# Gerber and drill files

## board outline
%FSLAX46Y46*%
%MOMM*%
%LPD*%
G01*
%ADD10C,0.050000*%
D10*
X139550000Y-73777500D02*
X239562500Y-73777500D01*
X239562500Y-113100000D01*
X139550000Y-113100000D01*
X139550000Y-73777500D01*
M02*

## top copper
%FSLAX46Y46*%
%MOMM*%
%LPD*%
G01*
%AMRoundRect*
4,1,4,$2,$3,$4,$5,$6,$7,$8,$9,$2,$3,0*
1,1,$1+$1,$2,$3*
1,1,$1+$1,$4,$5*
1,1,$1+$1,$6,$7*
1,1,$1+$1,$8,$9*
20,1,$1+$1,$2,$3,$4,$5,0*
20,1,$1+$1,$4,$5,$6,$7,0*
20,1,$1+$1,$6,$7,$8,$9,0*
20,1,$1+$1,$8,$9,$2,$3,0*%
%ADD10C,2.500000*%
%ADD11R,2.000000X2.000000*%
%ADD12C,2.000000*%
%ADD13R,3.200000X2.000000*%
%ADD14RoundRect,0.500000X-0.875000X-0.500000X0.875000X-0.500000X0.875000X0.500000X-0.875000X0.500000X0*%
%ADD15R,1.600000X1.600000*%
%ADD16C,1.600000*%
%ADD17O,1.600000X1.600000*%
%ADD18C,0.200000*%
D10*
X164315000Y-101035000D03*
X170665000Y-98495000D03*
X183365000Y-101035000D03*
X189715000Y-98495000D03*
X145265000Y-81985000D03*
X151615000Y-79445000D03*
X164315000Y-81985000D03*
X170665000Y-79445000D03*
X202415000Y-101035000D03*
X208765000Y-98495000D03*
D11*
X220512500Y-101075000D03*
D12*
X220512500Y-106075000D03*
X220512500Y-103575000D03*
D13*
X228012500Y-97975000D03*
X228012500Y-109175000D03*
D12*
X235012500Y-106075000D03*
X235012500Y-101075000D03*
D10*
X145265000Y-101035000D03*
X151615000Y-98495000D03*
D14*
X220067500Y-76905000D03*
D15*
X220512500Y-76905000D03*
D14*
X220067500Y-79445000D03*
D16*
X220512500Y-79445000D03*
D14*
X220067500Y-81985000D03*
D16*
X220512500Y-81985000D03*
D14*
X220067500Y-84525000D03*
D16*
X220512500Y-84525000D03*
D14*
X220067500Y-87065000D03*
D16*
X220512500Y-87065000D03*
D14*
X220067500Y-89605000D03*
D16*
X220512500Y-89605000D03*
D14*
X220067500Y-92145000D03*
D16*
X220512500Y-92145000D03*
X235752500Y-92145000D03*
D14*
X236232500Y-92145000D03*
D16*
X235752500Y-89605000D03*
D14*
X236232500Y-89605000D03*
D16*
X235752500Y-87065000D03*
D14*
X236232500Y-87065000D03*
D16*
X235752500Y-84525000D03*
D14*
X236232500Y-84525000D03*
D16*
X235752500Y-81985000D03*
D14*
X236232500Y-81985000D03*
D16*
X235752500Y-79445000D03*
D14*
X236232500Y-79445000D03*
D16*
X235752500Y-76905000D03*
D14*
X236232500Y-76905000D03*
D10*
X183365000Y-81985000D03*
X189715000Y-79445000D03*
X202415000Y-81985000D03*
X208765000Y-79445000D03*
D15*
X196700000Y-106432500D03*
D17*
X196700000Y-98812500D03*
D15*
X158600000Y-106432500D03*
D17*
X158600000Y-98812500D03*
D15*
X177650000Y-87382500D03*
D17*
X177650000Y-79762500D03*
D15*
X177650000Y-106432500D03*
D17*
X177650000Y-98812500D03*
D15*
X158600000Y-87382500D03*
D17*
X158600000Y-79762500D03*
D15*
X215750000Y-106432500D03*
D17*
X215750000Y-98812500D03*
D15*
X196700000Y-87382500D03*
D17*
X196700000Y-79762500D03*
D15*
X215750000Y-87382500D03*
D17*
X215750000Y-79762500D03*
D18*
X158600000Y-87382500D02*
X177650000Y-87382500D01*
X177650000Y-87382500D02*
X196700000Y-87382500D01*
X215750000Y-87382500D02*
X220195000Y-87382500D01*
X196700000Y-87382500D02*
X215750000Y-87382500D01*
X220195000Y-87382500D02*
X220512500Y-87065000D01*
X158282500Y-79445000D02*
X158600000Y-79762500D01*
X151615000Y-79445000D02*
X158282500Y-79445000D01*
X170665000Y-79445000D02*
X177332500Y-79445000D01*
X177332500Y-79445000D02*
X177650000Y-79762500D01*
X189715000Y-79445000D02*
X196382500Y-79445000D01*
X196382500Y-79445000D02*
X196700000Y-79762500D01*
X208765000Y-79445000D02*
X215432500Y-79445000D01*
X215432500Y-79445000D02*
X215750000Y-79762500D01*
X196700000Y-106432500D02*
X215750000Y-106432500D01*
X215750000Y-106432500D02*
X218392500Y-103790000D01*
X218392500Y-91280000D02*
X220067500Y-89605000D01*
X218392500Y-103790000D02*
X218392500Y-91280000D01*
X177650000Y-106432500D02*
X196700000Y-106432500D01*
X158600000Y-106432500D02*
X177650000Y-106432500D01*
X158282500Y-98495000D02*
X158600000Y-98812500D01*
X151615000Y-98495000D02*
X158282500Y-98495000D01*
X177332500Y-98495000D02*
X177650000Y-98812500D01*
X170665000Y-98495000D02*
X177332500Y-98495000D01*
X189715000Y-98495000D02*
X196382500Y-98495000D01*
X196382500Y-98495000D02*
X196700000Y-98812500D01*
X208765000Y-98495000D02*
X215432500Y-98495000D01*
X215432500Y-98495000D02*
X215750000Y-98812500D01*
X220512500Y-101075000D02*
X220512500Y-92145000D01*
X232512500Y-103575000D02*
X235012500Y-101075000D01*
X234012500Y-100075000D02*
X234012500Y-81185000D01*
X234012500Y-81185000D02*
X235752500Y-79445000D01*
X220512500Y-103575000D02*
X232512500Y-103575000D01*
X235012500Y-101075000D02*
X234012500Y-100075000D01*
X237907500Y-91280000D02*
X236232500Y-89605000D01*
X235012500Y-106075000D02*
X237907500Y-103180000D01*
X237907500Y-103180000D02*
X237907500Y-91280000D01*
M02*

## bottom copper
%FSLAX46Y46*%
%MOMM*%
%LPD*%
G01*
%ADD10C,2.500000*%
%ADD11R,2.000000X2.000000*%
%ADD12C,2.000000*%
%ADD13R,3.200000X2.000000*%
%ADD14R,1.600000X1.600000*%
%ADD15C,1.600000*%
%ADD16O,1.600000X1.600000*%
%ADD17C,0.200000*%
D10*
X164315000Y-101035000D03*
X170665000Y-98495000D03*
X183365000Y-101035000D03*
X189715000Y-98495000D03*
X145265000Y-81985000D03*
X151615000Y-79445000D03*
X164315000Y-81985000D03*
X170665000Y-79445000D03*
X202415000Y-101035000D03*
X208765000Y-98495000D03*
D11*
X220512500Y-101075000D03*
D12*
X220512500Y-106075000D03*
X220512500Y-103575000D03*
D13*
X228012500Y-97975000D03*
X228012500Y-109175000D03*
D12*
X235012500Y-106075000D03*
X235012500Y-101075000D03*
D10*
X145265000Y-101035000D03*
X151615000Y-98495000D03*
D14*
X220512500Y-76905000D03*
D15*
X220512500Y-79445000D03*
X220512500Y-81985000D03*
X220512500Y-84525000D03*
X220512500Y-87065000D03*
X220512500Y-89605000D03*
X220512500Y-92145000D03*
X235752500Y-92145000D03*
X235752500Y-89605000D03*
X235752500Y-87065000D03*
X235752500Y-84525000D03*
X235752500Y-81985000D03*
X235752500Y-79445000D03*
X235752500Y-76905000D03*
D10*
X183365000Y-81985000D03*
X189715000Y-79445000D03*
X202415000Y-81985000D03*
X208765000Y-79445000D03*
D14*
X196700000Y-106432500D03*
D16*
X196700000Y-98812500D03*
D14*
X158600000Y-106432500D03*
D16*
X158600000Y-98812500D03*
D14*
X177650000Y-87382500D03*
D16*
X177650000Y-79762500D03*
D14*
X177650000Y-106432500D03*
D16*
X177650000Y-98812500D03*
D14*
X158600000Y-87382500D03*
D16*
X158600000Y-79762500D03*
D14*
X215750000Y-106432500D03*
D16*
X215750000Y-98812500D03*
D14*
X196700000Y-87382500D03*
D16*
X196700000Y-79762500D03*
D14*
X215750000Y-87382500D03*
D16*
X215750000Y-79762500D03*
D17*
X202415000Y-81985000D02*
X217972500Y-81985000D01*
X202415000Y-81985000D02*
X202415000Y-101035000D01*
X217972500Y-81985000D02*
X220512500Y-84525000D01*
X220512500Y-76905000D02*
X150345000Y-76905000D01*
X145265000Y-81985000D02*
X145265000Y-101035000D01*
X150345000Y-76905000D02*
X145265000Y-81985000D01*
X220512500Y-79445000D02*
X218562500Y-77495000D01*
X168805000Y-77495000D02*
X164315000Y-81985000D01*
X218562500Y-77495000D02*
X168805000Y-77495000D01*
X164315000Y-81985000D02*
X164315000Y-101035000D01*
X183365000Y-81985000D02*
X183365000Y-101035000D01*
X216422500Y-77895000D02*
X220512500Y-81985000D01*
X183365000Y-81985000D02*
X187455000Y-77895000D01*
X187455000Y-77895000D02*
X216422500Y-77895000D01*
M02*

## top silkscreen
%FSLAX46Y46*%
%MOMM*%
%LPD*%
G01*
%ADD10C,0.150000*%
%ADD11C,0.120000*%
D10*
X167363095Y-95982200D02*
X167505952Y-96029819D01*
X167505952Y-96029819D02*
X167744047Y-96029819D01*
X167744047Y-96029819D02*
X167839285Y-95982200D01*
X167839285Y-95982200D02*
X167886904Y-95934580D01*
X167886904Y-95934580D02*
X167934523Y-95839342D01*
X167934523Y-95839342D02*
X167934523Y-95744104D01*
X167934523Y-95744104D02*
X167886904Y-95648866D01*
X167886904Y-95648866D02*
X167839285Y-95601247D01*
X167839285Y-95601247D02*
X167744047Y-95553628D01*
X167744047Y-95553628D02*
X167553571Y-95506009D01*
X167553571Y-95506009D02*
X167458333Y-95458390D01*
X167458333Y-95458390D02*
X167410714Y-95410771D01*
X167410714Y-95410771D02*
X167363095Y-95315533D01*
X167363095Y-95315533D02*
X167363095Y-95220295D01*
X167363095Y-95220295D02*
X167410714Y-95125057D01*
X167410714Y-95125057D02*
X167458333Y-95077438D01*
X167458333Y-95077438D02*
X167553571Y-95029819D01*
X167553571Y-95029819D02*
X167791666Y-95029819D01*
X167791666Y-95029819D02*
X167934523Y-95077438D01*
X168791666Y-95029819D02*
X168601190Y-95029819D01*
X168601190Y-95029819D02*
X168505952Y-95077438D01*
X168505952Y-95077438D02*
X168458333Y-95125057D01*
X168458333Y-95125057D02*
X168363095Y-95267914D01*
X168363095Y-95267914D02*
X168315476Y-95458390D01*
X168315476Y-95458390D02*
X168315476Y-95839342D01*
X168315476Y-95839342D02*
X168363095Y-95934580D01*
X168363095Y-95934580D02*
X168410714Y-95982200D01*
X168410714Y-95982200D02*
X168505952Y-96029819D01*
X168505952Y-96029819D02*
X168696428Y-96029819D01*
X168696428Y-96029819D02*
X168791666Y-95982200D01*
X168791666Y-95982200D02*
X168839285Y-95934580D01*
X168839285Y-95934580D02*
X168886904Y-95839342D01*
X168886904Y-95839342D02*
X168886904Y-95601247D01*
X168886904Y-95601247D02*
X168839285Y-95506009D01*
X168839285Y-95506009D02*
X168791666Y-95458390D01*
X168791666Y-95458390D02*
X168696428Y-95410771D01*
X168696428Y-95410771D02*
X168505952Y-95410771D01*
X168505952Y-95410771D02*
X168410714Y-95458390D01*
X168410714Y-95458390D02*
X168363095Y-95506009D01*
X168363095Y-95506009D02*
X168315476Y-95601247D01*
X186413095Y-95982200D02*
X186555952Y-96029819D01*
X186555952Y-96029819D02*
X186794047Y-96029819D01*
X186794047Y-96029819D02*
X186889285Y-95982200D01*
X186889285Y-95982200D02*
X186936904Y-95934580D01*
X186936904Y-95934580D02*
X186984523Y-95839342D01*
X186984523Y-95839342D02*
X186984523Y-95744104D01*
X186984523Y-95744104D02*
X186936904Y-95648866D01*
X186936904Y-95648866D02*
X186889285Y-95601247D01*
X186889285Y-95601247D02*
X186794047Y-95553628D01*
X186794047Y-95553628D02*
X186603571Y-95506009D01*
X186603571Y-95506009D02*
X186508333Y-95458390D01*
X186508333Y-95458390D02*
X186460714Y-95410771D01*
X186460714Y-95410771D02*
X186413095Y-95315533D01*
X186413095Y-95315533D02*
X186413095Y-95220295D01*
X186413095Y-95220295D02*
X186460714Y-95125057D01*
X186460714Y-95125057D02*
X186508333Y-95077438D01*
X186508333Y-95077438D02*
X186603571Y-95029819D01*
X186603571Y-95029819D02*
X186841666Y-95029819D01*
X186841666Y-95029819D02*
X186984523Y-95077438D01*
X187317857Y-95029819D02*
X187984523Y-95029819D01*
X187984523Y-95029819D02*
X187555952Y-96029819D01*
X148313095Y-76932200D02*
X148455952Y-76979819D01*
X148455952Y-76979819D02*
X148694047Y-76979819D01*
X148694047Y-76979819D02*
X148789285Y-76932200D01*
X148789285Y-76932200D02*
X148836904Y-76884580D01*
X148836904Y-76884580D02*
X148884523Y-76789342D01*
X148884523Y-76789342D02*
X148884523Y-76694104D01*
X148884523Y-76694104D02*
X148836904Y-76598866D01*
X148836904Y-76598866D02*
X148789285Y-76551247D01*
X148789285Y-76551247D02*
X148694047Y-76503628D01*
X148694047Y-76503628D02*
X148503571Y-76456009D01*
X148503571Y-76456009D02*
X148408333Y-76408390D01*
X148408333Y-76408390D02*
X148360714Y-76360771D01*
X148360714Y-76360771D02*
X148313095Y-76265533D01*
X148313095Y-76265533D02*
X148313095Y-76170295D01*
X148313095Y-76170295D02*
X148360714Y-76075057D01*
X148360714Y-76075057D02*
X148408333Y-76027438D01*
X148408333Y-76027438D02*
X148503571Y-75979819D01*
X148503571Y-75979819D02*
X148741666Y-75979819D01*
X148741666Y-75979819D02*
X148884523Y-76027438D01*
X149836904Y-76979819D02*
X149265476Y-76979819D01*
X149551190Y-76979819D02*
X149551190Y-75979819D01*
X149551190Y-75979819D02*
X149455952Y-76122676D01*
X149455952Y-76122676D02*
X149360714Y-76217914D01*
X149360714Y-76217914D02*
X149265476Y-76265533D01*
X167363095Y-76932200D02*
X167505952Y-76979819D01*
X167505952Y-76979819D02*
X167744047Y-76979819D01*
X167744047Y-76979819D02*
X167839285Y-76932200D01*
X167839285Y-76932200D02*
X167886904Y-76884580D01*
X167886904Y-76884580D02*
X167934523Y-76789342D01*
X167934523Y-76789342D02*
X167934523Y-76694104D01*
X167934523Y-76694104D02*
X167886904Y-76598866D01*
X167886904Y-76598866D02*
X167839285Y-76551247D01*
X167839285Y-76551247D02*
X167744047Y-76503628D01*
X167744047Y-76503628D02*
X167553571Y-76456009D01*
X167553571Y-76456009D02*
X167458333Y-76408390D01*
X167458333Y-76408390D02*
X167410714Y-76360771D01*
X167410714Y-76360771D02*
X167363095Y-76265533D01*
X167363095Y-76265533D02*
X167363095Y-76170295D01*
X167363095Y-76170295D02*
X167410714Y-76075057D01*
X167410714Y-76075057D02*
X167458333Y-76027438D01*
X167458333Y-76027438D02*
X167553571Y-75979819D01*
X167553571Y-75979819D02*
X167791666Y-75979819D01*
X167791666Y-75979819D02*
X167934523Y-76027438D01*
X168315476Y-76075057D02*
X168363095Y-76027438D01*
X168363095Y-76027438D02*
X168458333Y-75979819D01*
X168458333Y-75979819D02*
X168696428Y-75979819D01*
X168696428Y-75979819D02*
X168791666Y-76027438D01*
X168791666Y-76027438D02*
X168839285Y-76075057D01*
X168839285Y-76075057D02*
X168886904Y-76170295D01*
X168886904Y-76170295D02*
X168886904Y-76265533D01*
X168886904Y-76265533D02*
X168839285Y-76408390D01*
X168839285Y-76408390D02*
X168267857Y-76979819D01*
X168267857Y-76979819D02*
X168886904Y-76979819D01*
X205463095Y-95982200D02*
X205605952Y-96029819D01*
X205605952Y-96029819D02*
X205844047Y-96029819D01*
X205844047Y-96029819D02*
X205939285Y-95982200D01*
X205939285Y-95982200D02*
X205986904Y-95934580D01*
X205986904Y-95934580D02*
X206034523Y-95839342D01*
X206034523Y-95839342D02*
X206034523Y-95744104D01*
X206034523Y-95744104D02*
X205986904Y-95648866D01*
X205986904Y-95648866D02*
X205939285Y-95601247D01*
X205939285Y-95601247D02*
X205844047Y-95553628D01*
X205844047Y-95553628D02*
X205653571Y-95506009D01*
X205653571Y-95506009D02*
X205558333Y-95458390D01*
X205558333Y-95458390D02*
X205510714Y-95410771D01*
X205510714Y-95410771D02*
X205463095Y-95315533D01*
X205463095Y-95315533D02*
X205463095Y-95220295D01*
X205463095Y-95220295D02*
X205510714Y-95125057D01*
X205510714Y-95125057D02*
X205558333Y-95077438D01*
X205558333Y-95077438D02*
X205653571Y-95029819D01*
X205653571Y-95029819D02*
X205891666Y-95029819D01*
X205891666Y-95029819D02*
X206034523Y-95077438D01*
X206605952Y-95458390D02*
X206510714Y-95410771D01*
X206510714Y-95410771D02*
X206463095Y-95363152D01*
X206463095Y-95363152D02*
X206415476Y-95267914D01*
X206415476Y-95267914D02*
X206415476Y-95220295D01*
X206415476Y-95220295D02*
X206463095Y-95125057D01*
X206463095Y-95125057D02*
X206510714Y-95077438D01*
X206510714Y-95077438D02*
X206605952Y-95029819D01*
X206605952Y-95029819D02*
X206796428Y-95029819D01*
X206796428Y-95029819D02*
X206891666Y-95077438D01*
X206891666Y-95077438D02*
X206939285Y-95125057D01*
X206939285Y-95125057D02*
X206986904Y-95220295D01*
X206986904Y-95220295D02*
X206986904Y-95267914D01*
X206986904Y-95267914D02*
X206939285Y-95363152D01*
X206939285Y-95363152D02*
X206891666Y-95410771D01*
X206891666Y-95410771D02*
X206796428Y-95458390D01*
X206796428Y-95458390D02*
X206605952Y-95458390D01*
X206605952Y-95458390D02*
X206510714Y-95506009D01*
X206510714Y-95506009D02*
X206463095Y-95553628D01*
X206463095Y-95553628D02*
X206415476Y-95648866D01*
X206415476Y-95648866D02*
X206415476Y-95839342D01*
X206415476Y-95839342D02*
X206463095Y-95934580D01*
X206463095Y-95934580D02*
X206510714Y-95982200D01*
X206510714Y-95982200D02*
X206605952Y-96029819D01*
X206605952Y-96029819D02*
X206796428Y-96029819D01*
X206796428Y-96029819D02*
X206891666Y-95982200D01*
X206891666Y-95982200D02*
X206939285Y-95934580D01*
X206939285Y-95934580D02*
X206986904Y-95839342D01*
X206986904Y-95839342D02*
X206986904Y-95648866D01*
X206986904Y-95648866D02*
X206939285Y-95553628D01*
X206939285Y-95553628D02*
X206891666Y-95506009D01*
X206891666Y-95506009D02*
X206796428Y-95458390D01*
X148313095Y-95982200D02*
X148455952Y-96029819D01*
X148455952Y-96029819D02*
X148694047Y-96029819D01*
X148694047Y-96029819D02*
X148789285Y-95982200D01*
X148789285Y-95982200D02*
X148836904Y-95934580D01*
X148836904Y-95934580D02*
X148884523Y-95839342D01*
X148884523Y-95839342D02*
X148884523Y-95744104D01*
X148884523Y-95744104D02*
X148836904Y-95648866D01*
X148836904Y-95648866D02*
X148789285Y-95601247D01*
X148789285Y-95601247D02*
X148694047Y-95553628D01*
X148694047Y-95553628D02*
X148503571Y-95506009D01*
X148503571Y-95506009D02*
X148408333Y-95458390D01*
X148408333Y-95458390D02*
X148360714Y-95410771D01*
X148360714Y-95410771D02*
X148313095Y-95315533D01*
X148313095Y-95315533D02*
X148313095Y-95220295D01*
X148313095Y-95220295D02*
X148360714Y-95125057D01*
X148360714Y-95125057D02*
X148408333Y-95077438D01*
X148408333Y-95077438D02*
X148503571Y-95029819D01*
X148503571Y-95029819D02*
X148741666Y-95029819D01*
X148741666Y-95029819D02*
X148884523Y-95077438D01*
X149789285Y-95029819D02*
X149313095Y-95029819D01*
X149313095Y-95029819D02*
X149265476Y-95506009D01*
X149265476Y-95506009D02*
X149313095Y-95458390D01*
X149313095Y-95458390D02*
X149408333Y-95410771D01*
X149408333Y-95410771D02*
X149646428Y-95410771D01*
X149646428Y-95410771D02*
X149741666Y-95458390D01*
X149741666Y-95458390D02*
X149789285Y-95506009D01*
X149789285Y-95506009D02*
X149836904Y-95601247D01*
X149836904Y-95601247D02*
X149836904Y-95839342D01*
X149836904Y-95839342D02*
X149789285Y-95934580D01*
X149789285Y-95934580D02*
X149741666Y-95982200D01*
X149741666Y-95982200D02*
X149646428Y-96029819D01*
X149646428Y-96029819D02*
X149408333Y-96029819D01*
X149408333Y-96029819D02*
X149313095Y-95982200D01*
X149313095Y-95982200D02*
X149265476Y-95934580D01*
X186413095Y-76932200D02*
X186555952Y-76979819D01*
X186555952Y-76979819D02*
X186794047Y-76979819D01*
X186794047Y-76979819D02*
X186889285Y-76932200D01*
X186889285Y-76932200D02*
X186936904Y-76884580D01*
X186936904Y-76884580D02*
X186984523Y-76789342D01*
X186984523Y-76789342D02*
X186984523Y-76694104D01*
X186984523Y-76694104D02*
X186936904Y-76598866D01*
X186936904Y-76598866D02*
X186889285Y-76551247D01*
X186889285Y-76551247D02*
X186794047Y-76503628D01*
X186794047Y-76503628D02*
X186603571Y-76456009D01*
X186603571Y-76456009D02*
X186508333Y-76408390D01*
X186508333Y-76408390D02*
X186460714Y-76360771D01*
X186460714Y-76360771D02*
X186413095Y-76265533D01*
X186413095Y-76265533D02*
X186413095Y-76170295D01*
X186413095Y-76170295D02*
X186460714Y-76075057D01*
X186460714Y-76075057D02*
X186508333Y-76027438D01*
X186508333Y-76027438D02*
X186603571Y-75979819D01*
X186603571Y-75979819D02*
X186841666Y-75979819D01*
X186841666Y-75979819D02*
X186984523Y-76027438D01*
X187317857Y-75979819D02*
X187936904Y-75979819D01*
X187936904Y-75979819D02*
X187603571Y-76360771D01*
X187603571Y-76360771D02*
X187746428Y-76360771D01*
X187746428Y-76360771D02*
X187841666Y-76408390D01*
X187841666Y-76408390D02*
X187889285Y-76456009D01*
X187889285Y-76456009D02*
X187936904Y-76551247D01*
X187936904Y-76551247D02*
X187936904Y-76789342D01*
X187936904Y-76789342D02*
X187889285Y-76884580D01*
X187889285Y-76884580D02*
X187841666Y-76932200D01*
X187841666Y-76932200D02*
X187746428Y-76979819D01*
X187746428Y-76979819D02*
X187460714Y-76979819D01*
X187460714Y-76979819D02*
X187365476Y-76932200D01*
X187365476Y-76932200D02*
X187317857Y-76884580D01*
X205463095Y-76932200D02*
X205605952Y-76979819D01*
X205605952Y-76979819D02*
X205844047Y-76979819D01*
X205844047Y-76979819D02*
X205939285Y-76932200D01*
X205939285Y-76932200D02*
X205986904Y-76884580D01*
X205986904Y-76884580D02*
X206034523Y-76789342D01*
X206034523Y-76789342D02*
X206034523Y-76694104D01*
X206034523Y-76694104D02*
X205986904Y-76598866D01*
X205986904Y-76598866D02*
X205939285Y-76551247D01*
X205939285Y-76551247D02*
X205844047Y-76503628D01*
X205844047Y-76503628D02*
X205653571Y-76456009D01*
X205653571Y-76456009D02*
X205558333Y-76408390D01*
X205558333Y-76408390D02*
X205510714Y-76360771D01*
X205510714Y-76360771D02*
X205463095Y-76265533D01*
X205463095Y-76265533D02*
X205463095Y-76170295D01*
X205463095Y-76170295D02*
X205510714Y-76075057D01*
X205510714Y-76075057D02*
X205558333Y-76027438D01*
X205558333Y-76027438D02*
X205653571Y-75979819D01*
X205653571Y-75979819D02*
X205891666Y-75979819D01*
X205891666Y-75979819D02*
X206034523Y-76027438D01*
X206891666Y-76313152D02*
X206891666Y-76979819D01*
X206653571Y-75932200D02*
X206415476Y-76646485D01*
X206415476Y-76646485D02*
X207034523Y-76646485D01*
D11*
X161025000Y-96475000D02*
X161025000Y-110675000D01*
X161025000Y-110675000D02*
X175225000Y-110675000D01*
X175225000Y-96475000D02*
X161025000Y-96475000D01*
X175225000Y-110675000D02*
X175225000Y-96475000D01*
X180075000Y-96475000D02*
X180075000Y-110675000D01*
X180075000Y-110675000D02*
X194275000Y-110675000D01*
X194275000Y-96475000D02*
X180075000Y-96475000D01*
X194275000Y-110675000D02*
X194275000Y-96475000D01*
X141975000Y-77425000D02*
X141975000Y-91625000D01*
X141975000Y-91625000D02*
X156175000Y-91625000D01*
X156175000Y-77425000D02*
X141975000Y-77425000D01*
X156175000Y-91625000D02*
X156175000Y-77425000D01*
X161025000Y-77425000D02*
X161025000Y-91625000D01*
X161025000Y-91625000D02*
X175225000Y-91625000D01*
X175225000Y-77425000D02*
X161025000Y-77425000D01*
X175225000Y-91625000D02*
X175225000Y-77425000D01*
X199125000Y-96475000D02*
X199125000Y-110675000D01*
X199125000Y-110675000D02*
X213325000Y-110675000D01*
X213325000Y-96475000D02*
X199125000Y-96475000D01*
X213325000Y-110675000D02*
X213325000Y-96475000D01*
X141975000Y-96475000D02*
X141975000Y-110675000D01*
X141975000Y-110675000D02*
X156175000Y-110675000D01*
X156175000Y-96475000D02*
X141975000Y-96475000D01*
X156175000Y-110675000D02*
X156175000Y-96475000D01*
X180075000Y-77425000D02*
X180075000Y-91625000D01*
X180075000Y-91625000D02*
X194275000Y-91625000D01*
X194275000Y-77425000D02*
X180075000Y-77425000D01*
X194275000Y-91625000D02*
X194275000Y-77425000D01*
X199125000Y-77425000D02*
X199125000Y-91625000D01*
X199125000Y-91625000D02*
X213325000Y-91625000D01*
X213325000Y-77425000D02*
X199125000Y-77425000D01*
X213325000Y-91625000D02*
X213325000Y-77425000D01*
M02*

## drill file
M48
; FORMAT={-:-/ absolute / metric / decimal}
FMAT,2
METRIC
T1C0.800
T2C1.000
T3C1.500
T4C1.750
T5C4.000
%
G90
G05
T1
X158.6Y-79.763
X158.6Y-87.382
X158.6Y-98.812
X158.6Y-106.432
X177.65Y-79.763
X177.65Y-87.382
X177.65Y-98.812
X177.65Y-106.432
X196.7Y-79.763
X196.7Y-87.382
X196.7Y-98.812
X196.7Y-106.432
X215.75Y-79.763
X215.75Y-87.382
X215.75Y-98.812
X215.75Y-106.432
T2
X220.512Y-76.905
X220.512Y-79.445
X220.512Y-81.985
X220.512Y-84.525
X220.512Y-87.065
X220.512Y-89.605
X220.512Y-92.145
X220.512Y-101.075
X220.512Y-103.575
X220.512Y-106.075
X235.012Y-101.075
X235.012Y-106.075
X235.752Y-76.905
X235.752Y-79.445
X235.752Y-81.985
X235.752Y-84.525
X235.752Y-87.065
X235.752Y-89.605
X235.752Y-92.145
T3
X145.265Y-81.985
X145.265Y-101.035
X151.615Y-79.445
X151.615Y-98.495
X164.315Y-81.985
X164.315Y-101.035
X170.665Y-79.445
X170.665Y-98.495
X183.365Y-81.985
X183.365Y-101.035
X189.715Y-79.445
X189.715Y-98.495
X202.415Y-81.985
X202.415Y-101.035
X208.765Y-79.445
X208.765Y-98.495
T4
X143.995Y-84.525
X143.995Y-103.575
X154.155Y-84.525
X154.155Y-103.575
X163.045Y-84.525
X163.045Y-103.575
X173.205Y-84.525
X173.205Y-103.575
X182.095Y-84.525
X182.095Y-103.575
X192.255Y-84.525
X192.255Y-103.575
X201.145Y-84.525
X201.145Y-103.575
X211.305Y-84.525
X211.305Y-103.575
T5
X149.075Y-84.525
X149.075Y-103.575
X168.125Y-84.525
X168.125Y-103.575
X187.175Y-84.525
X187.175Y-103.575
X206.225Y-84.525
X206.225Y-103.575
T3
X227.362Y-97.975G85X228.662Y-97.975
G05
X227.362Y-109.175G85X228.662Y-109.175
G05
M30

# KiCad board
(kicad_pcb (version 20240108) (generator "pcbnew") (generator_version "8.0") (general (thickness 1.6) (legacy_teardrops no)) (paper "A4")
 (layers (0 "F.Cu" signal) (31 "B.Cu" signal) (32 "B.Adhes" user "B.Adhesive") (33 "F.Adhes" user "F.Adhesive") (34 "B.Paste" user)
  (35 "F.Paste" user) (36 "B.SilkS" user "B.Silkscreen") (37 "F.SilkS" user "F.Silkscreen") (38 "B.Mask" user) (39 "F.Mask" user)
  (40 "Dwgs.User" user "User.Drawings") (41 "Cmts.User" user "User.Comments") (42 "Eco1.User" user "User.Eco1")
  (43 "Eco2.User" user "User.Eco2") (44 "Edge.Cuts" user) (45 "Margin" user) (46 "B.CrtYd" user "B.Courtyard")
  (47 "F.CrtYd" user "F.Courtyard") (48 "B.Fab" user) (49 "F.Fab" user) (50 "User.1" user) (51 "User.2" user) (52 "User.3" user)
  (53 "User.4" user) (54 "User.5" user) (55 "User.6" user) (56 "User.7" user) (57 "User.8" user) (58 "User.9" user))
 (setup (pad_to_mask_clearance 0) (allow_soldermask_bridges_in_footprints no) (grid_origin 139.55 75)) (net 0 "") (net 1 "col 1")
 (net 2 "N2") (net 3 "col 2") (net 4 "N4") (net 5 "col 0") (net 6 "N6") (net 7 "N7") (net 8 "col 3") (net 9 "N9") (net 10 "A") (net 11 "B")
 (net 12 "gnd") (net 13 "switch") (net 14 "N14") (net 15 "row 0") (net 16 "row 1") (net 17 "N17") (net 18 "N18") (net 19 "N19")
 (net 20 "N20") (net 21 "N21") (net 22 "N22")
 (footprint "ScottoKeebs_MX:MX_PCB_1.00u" (layer "F.Cu") (at 168.125 103.575)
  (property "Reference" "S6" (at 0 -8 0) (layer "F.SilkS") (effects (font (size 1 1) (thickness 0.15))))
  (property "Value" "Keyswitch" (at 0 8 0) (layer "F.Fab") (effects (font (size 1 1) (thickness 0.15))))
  (fp_line (start -7.1 -7.1) (end -7.1 7.1) (stroke (width 0.12) (type solid)) (layer "F.SilkS"))
  (fp_line (start -7.1 7.1) (end 7.1 7.1) (stroke (width 0.12) (type solid)) (layer "F.SilkS"))
  (fp_line (start 7.1 -7.1) (end -7.1 -7.1) (stroke (width 0.12) (type solid)) (layer "F.SilkS"))
  (fp_line (start 7.1 7.1) (end 7.1 -7.1) (stroke (width 0.12) (type solid)) (layer "F.SilkS"))
  (pad "" np_thru_hole circle (at -5.08 0) (size 1.75 1.75) (drill 1.75) (layers "*.Cu" "*.Mask"))
  (pad "" np_thru_hole circle (at 0 0) (size 4 4) (drill 4) (layers "*.Cu" "*.Mask"))
  (pad "" np_thru_hole circle (at 5.08 0) (size 1.75 1.75) (drill 1.75) (layers "*.Cu" "*.Mask"))
  (pad "1" thru_hole circle (at -3.81 -2.54) (size 2.5 2.5) (drill 1.5) (layers "*.Cu" "*.Mask") (remove_unused_layers no) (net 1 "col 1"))
  (pad "2" thru_hole circle (at 2.54 -5.08) (size 2.5 2.5) (drill 1.5) (layers "*.Cu" "*.Mask") (remove_unused_layers no) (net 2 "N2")))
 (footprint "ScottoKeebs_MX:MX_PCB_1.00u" (layer "F.Cu") (at 187.175 103.575)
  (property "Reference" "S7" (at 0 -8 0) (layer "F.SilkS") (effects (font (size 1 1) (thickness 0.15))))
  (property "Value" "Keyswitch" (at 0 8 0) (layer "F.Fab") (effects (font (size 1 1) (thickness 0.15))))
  (fp_line (start -7.1 -7.1) (end -7.1 7.1) (stroke (width 0.12) (type solid)) (layer "F.SilkS"))
  (fp_line (start -7.1 7.1) (end 7.1 7.1) (stroke (width 0.12) (type solid)) (layer "F.SilkS"))
  (fp_line (start 7.1 -7.1) (end -7.1 -7.1) (stroke (width 0.12) (type solid)) (layer "F.SilkS"))
  (fp_line (start 7.1 7.1) (end 7.1 -7.1) (stroke (width 0.12) (type solid)) (layer "F.SilkS"))
  (pad "" np_thru_hole circle (at -5.08 0) (size 1.75 1.75) (drill 1.75) (layers "*.Cu" "*.Mask"))
  (pad "" np_thru_hole circle (at 0 0) (size 4 4) (drill 4) (layers "*.Cu" "*.Mask"))
  (pad "" np_thru_hole circle (at 5.08 0) (size 1.75 1.75) (drill 1.75) (layers "*.Cu" "*.Mask"))
  (pad "1" thru_hole circle (at -3.81 -2.54) (size 2.5 2.5) (drill 1.5) (layers "*.Cu" "*.Mask") (remove_unused_layers no) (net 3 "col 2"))
  (pad "2" thru_hole circle (at 2.54 -5.08) (size 2.5 2.5) (drill 1.5) (layers "*.Cu" "*.Mask") (remove_unused_layers no) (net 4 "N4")))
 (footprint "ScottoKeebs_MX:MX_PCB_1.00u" (layer "F.Cu") (at 149.075 84.525)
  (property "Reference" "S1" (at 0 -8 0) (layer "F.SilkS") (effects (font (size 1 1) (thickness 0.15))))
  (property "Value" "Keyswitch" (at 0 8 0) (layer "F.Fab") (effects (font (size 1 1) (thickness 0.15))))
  (fp_line (start -7.1 -7.1) (end -7.1 7.1) (stroke (width 0.12) (type solid)) (layer "F.SilkS"))
  (fp_line (start -7.1 7.1) (end 7.1 7.1) (stroke (width 0.12) (type solid)) (layer "F.SilkS"))
  (fp_line (start 7.1 -7.1) (end -7.1 -7.1) (stroke (width 0.12) (type solid)) (layer "F.SilkS"))
  (fp_line (start 7.1 7.1) (end 7.1 -7.1) (stroke (width 0.12) (type solid)) (layer "F.SilkS"))
  (pad "" np_thru_hole circle (at -5.08 0) (size 1.75 1.75) (drill 1.75) (layers "*.Cu" "*.Mask"))
  (pad "" np_thru_hole circle (at 0 0) (size 4 4) (drill 4) (layers "*.Cu" "*.Mask"))
  (pad "" np_thru_hole circle (at 5.08 0) (size 1.75 1.75) (drill 1.75) (layers "*.Cu" "*.Mask"))
  (pad "1" thru_hole circle (at -3.81 -2.54) (size 2.5 2.5) (drill 1.5) (layers "*.Cu" "*.Mask") (remove_unused_layers no) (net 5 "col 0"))
  (pad "2" thru_hole circle (at 2.54 -5.08) (size 2.5 2.5) (drill 1.5) (layers "*.Cu" "*.Mask") (remove_unused_layers no) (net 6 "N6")))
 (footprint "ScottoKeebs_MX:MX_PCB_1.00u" (layer "F.Cu") (at 168.125 84.525)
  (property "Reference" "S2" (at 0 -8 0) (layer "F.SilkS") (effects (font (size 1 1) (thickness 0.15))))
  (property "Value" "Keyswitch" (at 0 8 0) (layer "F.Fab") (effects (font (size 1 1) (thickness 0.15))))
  (fp_line (start -7.1 -7.1) (end -7.1 7.1) (stroke (width 0.12) (type solid)) (layer "F.SilkS"))
  (fp_line (start -7.1 7.1) (end 7.1 7.1) (stroke (width 0.12) (type solid)) (layer "F.SilkS"))
  (fp_line (start 7.1 -7.1) (end -7.1 -7.1) (stroke (width 0.12) (type solid)) (layer "F.SilkS"))
  (fp_line (start 7.1 7.1) (end 7.1 -7.1) (stroke (width 0.12) (type solid)) (layer "F.SilkS"))
  (pad "" np_thru_hole circle (at -5.08 0) (size 1.75 1.75) (drill 1.75) (layers "*.Cu" "*.Mask"))
  (pad "" np_thru_hole circle (at 0 0) (size 4 4) (drill 4) (layers "*.Cu" "*.Mask"))
  (pad "" np_thru_hole circle (at 5.08 0) (size 1.75 1.75) (drill 1.75) (layers "*.Cu" "*.Mask"))
  (pad "1" thru_hole circle (at -3.81 -2.54) (size 2.5 2.5) (drill 1.5) (layers "*.Cu" "*.Mask") (remove_unused_layers no) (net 1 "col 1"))
  (pad "2" thru_hole circle (at 2.54 -5.08) (size 2.5 2.5) (drill 1.5) (layers "*.Cu" "*.Mask") (remove_unused_layers no) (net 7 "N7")))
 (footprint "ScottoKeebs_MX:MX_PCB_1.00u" (layer "F.Cu") (at 206.225 103.575)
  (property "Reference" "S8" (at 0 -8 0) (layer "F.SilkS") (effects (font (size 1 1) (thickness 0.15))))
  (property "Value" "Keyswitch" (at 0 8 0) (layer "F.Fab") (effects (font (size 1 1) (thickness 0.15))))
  (fp_line (start -7.1 -7.1) (end -7.1 7.1) (stroke (width 0.12) (type solid)) (layer "F.SilkS"))
  (fp_line (start -7.1 7.1) (end 7.1 7.1) (stroke (width 0.12) (type solid)) (layer "F.SilkS"))
  (fp_line (start 7.1 -7.1) (end -7.1 -7.1) (stroke (width 0.12) (type solid)) (layer "F.SilkS"))
  (fp_line (start 7.1 7.1) (end 7.1 -7.1) (stroke (width 0.12) (type solid)) (layer "F.SilkS"))
  (pad "" np_thru_hole circle (at -5.08 0) (size 1.75 1.75) (drill 1.75) (layers "*.Cu" "*.Mask"))
  (pad "" np_thru_hole circle (at 0 0) (size 4 4) (drill 4) (layers "*.Cu" "*.Mask"))
  (pad "" np_thru_hole circle (at 5.08 0) (size 1.75 1.75) (drill 1.75) (layers "*.Cu" "*.Mask"))
  (pad "1" thru_hole circle (at -3.81 -2.54) (size 2.5 2.5) (drill 1.5) (layers "*.Cu" "*.Mask") (remove_unused_layers no) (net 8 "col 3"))
  (pad "2" thru_hole circle (at 2.54 -5.08) (size 2.5 2.5) (drill 1.5) (layers "*.Cu" "*.Mask") (remove_unused_layers no) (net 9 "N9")))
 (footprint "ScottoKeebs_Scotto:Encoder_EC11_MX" (layer "F.Cu") (at 228.0125 103.575)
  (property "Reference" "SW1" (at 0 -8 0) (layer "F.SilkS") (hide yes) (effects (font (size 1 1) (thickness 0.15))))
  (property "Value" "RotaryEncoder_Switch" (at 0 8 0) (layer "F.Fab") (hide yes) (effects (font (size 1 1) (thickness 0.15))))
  (pad "A" thru_hole rect (at -7.5 -2.5) (size 2 2) (drill 1) (layers "*.Cu" "*.Mask") (remove_unused_layers no) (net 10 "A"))
  (pad "B" thru_hole circle (at -7.5 2.5) (size 2 2) (drill 1) (layers "*.Cu" "*.Mask") (remove_unused_layers no) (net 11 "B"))
  (pad "C" thru_hole circle (at -7.5 0) (size 2 2) (drill 1) (layers "*.Cu" "*.Mask") (remove_unused_layers no) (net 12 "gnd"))
  (pad "MP" thru_hole rect (at 0 -5.6) (size 3.2 2) (drill oval 2.8 1.5) (layers "*.Cu" "*.Mask") (remove_unused_layers no))
  (pad "MP" thru_hole rect (at 0 5.6) (size 3.2 2) (drill oval 2.8 1.5) (layers "*.Cu" "*.Mask") (remove_unused_layers no))
  (pad "S1" thru_hole circle (at 7 2.5) (size 2 2) (drill 1) (layers "*.Cu" "*.Mask") (remove_unused_layers no) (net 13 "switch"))
  (pad "S2" thru_hole circle (at 7 -2.5) (size 2 2) (drill 1) (layers "*.Cu" "*.Mask") (remove_unused_layers no) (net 12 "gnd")))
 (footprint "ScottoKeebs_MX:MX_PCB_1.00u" (layer "F.Cu") (at 149.075 103.575)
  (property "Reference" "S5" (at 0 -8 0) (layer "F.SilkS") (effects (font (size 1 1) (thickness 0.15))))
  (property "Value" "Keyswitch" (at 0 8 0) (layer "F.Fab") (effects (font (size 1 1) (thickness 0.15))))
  (fp_line (start -7.1 -7.1) (end -7.1 7.1) (stroke (width 0.12) (type solid)) (layer "F.SilkS"))
  (fp_line (start -7.1 7.1) (end 7.1 7.1) (stroke (width 0.12) (type solid)) (layer "F.SilkS"))
  (fp_line (start 7.1 -7.1) (end -7.1 -7.1) (stroke (width 0.12) (type solid)) (layer "F.SilkS"))
  (fp_line (start 7.1 7.1) (end 7.1 -7.1) (stroke (width 0.12) (type solid)) (layer "F.SilkS"))
  (pad "" np_thru_hole circle (at -5.08 0) (size 1.75 1.75) (drill 1.75) (layers "*.Cu" "*.Mask"))
  (pad "" np_thru_hole circle (at 0 0) (size 4 4) (drill 4) (layers "*.Cu" "*.Mask"))
  (pad "" np_thru_hole circle (at 5.08 0) (size 1.75 1.75) (drill 1.75) (layers "*.Cu" "*.Mask"))
  (pad "1" thru_hole circle (at -3.81 -2.54) (size 2.5 2.5) (drill 1.5) (layers "*.Cu" "*.Mask") (remove_unused_layers no) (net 5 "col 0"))
  (pad "2" thru_hole circle (at 2.54 -5.08) (size 2.5 2.5) (drill 1.5) (layers "*.Cu" "*.Mask") (remove_unused_layers no) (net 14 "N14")))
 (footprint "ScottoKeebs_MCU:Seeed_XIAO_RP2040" (layer "F.Cu") (at 228.1325 84.525)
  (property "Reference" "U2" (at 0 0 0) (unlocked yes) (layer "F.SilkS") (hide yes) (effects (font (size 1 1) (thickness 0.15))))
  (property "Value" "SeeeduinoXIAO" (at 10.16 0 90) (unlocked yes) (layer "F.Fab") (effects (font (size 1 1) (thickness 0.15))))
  (pad "1" smd roundrect (at -8.065 -7.62) (size 2.75 2) (layers "F.Cu" "F.Paste" "F.Mask") (roundrect_rratio 0.25) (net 5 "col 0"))
  (pad "1" thru_hole rect (at -7.62 -7.62 90) (size 1.6 1.6) (drill 1) (layers "*.Cu" "*.Mask") (remove_unused_layers no) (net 5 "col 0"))
  (pad "2" smd roundrect (at -8.065 -5.08) (size 2.75 2) (layers "F.Cu" "F.Paste" "F.Mask") (roundrect_rratio 0.25) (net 1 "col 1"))
  (pad "2" thru_hole circle (at -7.62 -5.08 90) (size 1.6 1.6) (drill 1) (layers "*.Cu" "*.Mask") (remove_unused_layers no) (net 1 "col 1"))
  (pad "3" smd roundrect (at -8.065 -2.54) (size 2.75 2) (layers "F.Cu" "F.Paste" "F.Mask") (roundrect_rratio 0.25) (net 3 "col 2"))
  (pad "3" thru_hole circle (at -7.62 -2.54 90) (size 1.6 1.6) (drill 1) (layers "*.Cu" "*.Mask") (remove_unused_layers no) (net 3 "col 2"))
  (pad "4" smd roundrect (at -8.065 0) (size 2.75 2) (layers "F.Cu" "F.Paste" "F.Mask") (roundrect_rratio 0.25) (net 8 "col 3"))
  (pad "4" thru_hole circle (at -7.62 0 90) (size 1.6 1.6) (drill 1) (layers "*.Cu" "*.Mask") (remove_unused_layers no) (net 8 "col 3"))
  (pad "5" smd roundrect (at -8.065 2.54) (size 2.75 2) (layers "F.Cu" "F.Paste" "F.Mask") (roundrect_rratio 0.25) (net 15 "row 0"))
  (pad "5" thru_hole circle (at -7.62 2.54 90) (size 1.6 1.6) (drill 1) (layers "*.Cu" "*.Mask") (remove_unused_layers no) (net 15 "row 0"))
  (pad "6" smd roundrect (at -8.065 5.08) (size 2.75 2) (layers "F.Cu" "F.Paste" "F.Mask") (roundrect_rratio 0.25) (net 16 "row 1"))
  (pad "6" thru_hole circle (at -7.62 5.08 90) (size 1.6 1.6) (drill 1) (layers "*.Cu" "*.Mask") (remove_unused_layers no) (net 16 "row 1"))
  (pad "7" smd roundrect (at -8.065 7.62) (size 2.75 2) (layers "F.Cu" "F.Paste" "F.Mask") (roundrect_rratio 0.25) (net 10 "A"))
  (pad "7" thru_hole circle (at -7.62 7.62 90) (size 1.6 1.6) (drill 1) (layers "*.Cu" "*.Mask") (remove_unused_layers no) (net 10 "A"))
  (pad "8" thru_hole circle (at 7.62 7.62 90) (size 1.6 1.6) (drill 1) (layers "*.Cu" "*.Mask") (remove_unused_layers no) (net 11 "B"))
  (pad "8" smd roundrect (at 8.1 7.62) (size 2.75 2) (layers "F.Cu" "F.Paste" "F.Mask") (roundrect_rratio 0.25) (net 11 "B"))
  (pad "9" thru_hole circle (at 7.62 5.08 90) (size 1.6 1.6) (drill 1) (layers "*.Cu" "*.Mask") (remove_unused_layers no) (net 13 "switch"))
  (pad "9" smd roundrect (at 8.1 5.08) (size 2.75 2) (layers "F.Cu" "F.Paste" "F.Mask") (roundrect_rratio 0.25) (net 13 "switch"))
  (pad "10" thru_hole circle (at 7.62 2.54 90) (size 1.6 1.6) (drill 1) (layers "*.Cu" "*.Mask") (remove_unused_layers no) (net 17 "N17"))
  (pad "10" smd roundrect (at 8.1 2.54) (size 2.75 2) (layers "F.Cu" "F.Paste" "F.Mask") (roundrect_rratio 0.25) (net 17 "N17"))
  (pad "11" thru_hole circle (at 7.62 0 90) (size 1.6 1.6) (drill 1) (layers "*.Cu" "*.Mask") (remove_unused_layers no) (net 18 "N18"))
  (pad "11" smd roundrect (at 8.1 0) (size 2.75 2) (layers "F.Cu" "F.Paste" "F.Mask") (roundrect_rratio 0.25) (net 18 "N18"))
  (pad "12" thru_hole circle (at 7.62 -2.54 90) (size 1.6 1.6) (drill 1) (layers "*.Cu" "*.Mask") (remove_unused_layers no) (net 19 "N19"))
  (pad "12" smd roundrect (at 8.1 -2.54) (size 2.75 2) (layers "F.Cu" "F.Paste" "F.Mask") (roundrect_rratio 0.25) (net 19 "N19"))
  (pad "13" thru_hole circle (at 7.62 -5.08 90) (size 1.6 1.6) (drill 1) (layers "*.Cu" "*.Mask") (remove_unused_layers no) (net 12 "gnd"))
  (pad "13" smd roundrect (at 8.1 -5.08) (size 2.75 2) (layers "F.Cu" "F.Paste" "F.Mask") (roundrect_rratio 0.25) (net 12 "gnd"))
  (pad "14" thru_hole circle (at 7.62 -7.62 90) (size 1.6 1.6) (drill 1) (layers "*.Cu" "*.Mask") (remove_unused_layers no) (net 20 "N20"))
  (pad "14" smd roundrect (at 8.1 -7.62) (size 2.75 2) (layers "F.Cu" "F.Paste" "F.Mask") (roundrect_rratio 0.25) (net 20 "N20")))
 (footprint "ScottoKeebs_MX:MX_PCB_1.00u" (layer "F.Cu") (at 187.175 84.525)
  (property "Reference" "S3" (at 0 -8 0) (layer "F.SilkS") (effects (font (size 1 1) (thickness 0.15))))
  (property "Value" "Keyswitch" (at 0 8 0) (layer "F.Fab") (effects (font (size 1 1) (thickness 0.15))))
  (fp_line (start -7.1 -7.1) (end -7.1 7.1) (stroke (width 0.12) (type solid)) (layer "F.SilkS"))
  (fp_line (start -7.1 7.1) (end 7.1 7.1) (stroke (width 0.12) (type solid)) (layer "F.SilkS"))
  (fp_line (start 7.1 -7.1) (end -7.1 -7.1) (stroke (width 0.12) (type solid)) (layer "F.SilkS"))
  (fp_line (start 7.1 7.1) (end 7.1 -7.1) (stroke (width 0.12) (type solid)) (layer "F.SilkS"))
  (pad "" np_thru_hole circle (at -5.08 0) (size 1.75 1.75) (drill 1.75) (layers "*.Cu" "*.Mask"))
  (pad "" np_thru_hole circle (at 0 0) (size 4 4) (drill 4) (layers "*.Cu" "*.Mask"))
  (pad "" np_thru_hole circle (at 5.08 0) (size 1.75 1.75) (drill 1.75) (layers "*.Cu" "*.Mask"))
  (pad "1" thru_hole circle (at -3.81 -2.54) (size 2.5 2.5) (drill 1.5) (layers "*.Cu" "*.Mask") (remove_unused_layers no) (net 3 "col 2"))
  (pad "2" thru_hole circle (at 2.54 -5.08) (size 2.5 2.5) (drill 1.5) (layers "*.Cu" "*.Mask") (remove_unused_layers no) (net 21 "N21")))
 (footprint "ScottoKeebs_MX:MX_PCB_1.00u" (layer "F.Cu") (at 206.225 84.525)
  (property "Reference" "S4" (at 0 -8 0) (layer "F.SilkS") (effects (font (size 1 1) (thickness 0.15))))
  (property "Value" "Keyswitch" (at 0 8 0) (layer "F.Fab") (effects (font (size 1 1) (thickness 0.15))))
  (fp_line (start -7.1 -7.1) (end -7.1 7.1) (stroke (width 0.12) (type solid)) (layer "F.SilkS"))
  (fp_line (start -7.1 7.1) (end 7.1 7.1) (stroke (width 0.12) (type solid)) (layer "F.SilkS"))
  (fp_line (start 7.1 -7.1) (end -7.1 -7.1) (stroke (width 0.12) (type solid)) (layer "F.SilkS"))
  (fp_line (start 7.1 7.1) (end 7.1 -7.1) (stroke (width 0.12) (type solid)) (layer "F.SilkS"))
  (pad "" np_thru_hole circle (at -5.08 0) (size 1.75 1.75) (drill 1.75) (layers "*.Cu" "*.Mask"))
  (pad "" np_thru_hole circle (at 0 0) (size 4 4) (drill 4) (layers "*.Cu" "*.Mask"))
  (pad "" np_thru_hole circle (at 5.08 0) (size 1.75 1.75) (drill 1.75) (layers "*.Cu" "*.Mask"))
  (pad "1" thru_hole circle (at -3.81 -2.54) (size 2.5 2.5) (drill 1.5) (layers "*.Cu" "*.Mask") (remove_unused_layers no) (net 8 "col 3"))
  (pad "2" thru_hole circle (at 2.54 -5.08) (size 2.5 2.5) (drill 1.5) (layers "*.Cu" "*.Mask") (remove_unused_layers no) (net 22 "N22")))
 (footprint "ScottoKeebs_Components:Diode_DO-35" (layer "B.Cu") (at 196.7 106.4325 90)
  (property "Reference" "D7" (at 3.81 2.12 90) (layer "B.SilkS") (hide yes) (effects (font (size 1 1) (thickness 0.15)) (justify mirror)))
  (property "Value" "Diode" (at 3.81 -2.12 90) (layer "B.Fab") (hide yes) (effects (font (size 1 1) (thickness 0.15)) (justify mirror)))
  (pad "1" thru_hole rect (at 0 0 90) (size 1.6 1.6) (drill 0.8) (layers "*.Cu" "*.Mask") (remove_unused_layers no) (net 16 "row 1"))
  (pad "2" thru_hole oval (at 7.62 0 90) (size 1.6 1.6) (drill 0.8) (layers "*.Cu" "*.Mask") (remove_unused_layers no) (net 4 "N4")))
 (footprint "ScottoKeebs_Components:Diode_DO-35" (layer "B.Cu") (at 158.6 106.4325 90)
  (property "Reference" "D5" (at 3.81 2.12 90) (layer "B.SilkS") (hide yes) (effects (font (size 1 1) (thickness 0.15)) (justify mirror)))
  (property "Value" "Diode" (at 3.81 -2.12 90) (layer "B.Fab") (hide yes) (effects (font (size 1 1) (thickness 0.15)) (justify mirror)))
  (pad "1" thru_hole rect (at 0 0 90) (size 1.6 1.6) (drill 0.8) (layers "*.Cu" "*.Mask") (remove_unused_layers no) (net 16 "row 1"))
  (pad "2" thru_hole oval (at 7.62 0 90) (size 1.6 1.6) (drill 0.8) (layers "*.Cu" "*.Mask") (remove_unused_layers no) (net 14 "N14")))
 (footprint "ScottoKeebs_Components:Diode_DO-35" (layer "B.Cu") (at 177.65 87.3825 90)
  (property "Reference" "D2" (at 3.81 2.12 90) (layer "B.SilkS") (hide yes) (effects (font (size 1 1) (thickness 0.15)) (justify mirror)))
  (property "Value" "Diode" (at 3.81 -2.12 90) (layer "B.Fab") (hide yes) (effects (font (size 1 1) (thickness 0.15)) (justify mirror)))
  (pad "1" thru_hole rect (at 0 0 90) (size 1.6 1.6) (drill 0.8) (layers "*.Cu" "*.Mask") (remove_unused_layers no) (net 15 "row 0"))
  (pad "2" thru_hole oval (at 7.62 0 90) (size 1.6 1.6) (drill 0.8) (layers "*.Cu" "*.Mask") (remove_unused_layers no) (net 7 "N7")))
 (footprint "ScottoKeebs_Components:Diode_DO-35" (layer "B.Cu") (at 177.65 106.4325 90)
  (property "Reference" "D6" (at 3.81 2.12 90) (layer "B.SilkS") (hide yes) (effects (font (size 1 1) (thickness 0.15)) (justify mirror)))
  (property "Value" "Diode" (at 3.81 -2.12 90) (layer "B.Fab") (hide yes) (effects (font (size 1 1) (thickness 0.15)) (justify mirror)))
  (pad "1" thru_hole rect (at 0 0 90) (size 1.6 1.6) (drill 0.8) (layers "*.Cu" "*.Mask") (remove_unused_layers no) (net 16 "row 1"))
  (pad "2" thru_hole oval (at 7.62 0 90) (size 1.6 1.6) (drill 0.8) (layers "*.Cu" "*.Mask") (remove_unused_layers no) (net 2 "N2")))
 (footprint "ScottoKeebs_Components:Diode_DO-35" (layer "B.Cu") (at 158.6 87.3825 90)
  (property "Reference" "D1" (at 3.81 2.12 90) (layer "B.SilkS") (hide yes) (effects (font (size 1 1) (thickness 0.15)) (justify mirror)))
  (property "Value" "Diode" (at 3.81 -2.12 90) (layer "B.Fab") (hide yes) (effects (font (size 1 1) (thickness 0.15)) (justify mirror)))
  (pad "1" thru_hole rect (at 0 0 90) (size 1.6 1.6) (drill 0.8) (layers "*.Cu" "*.Mask") (remove_unused_layers no) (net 15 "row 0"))
  (pad "2" thru_hole oval (at 7.62 0 90) (size 1.6 1.6) (drill 0.8) (layers "*.Cu" "*.Mask") (remove_unused_layers no) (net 6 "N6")))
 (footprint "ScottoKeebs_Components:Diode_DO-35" (layer "B.Cu") (at 215.75 106.4325 90)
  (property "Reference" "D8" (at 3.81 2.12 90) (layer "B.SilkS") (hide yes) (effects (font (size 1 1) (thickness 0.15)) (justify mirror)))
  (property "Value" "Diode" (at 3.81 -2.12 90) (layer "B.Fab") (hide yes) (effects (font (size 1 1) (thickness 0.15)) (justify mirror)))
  (pad "1" thru_hole rect (at 0 0 90) (size 1.6 1.6) (drill 0.8) (layers "*.Cu" "*.Mask") (remove_unused_layers no) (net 16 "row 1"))
  (pad "2" thru_hole oval (at 7.62 0 90) (size 1.6 1.6) (drill 0.8) (layers "*.Cu" "*.Mask") (remove_unused_layers no) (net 9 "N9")))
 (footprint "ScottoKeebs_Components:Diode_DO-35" (layer "B.Cu") (at 196.7 87.3825 90)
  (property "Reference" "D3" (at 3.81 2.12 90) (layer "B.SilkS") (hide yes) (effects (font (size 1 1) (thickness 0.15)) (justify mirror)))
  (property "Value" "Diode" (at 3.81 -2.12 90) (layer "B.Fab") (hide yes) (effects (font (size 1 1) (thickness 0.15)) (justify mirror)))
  (pad "1" thru_hole rect (at 0 0 90) (size 1.6 1.6) (drill 0.8) (layers "*.Cu" "*.Mask") (remove_unused_layers no) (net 15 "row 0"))
  (pad "2" thru_hole oval (at 7.62 0 90) (size 1.6 1.6) (drill 0.8) (layers "*.Cu" "*.Mask") (remove_unused_layers no) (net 21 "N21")))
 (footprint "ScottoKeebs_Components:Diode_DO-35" (layer "B.Cu") (at 215.75 87.3825 90)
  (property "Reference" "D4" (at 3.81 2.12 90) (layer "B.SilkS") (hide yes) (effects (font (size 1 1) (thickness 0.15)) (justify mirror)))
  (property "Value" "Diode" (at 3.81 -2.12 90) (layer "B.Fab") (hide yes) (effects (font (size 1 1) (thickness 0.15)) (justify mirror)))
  (pad "1" thru_hole rect (at 0 0 90) (size 1.6 1.6) (drill 0.8) (layers "*.Cu" "*.Mask") (remove_unused_layers no) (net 15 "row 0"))
  (pad "2" thru_hole oval (at 7.62 0 90) (size 1.6 1.6) (drill 0.8) (layers "*.Cu" "*.Mask") (remove_unused_layers no) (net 22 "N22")))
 (gr_rect (start 139.55 73.7775) (end 239.5625 113.1) (stroke (width 0.05) (type default)) (fill none) (layer "Edge.Cuts"))
 (segment (start 158.6 87.3825) (end 177.65 87.3825) (width 0.2) (layer "F.Cu") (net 15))
 (segment (start 177.65 87.3825) (end 196.7 87.3825) (width 0.2) (layer "F.Cu") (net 15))
 (segment (start 215.75 87.3825) (end 220.195 87.3825) (width 0.2) (layer "F.Cu") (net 15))
 (segment (start 196.7 87.3825) (end 215.75 87.3825) (width 0.2) (layer "F.Cu") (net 15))
 (segment (start 220.195 87.3825) (end 220.5125 87.065) (width 0.2) (layer "F.Cu") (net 15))
 (segment (start 158.2825 79.445) (end 158.6 79.7625) (width 0.2) (layer "F.Cu") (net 6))
 (segment (start 151.615 79.445) (end 158.2825 79.445) (width 0.2) (layer "F.Cu") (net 6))
 (segment (start 170.665 79.445) (end 177.3325 79.445) (width 0.2) (layer "F.Cu") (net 7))
 (segment (start 177.3325 79.445) (end 177.65 79.7625) (width 0.2) (layer "F.Cu") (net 7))
 (segment (start 189.715 79.445) (end 196.3825 79.445) (width 0.2) (layer "F.Cu") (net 21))
 (segment (start 196.3825 79.445) (end 196.7 79.7625) (width 0.2) (layer "F.Cu") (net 21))
 (segment (start 208.765 79.445) (end 215.4325 79.445) (width 0.2) (layer "F.Cu") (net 22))
 (segment (start 215.4325 79.445) (end 215.75 79.7625) (width 0.2) (layer "F.Cu") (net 22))
 (segment (start 196.7 106.4325) (end 215.75 106.4325) (width 0.2) (layer "F.Cu") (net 16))
 (segment (start 215.75 106.4325) (end 218.3925 103.79) (width 0.2) (layer "F.Cu") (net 16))
 (segment (start 218.3925 91.28) (end 220.0675 89.605) (width 0.2) (layer "F.Cu") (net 16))
 (segment (start 218.3925 103.79) (end 218.3925 91.28) (width 0.2) (layer "F.Cu") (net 16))
 (segment (start 177.65 106.4325) (end 196.7 106.4325) (width 0.2) (layer "F.Cu") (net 16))
 (segment (start 158.6 106.4325) (end 177.65 106.4325) (width 0.2) (layer "F.Cu") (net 16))
 (segment (start 158.2825 98.495) (end 158.6 98.8125) (width 0.2) (layer "F.Cu") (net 14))
 (segment (start 151.615 98.495) (end 158.2825 98.495) (width 0.2) (layer "F.Cu") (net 14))
 (segment (start 177.3325 98.495) (end 177.65 98.8125) (width 0.2) (layer "F.Cu") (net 2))
 (segment (start 170.665 98.495) (end 177.3325 98.495) (width 0.2) (layer "F.Cu") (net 2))
 (segment (start 189.715 98.495) (end 196.3825 98.495) (width 0.2) (layer "F.Cu") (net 4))
 (segment (start 196.3825 98.495) (end 196.7 98.8125) (width 0.2) (layer "F.Cu") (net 4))
 (segment (start 202.415 81.985) (end 217.9725 81.985) (width 0.2) (layer "B.Cu") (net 8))
 (segment (start 202.415 81.985) (end 202.415 101.035) (width 0.2) (layer "B.Cu") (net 8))
 (segment (start 217.9725 81.985) (end 220.5125 84.525) (width 0.2) (layer "B.Cu") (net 8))
 (segment (start 208.765 98.495) (end 215.4325 98.495) (width 0.2) (layer "F.Cu") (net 9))
 (segment (start 215.4325 98.495) (end 215.75 98.8125) (width 0.2) (layer "F.Cu") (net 9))
 (segment (start 220.5125 76.905) (end 150.345 76.905) (width 0.2) (layer "B.Cu") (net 5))
 (segment (start 145.265 81.985) (end 145.265 101.035) (width 0.2) (layer "B.Cu") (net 5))
 (segment (start 150.345 76.905) (end 145.265 81.985) (width 0.2) (layer "B.Cu") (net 5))
 (segment (start 220.5125 79.445) (end 218.5625 77.495) (width 0.2) (layer "B.Cu") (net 1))
 (segment (start 168.805 77.495) (end 164.315 81.985) (width 0.2) (layer "B.Cu") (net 1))
 (segment (start 218.5625 77.495) (end 168.805 77.495) (width 0.2) (layer "B.Cu") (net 1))
 (segment (start 164.315 81.985) (end 164.315 101.035) (width 0.2) (layer "B.Cu") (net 1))
 (segment (start 183.365 81.985) (end 183.365 101.035) (width 0.2) (layer "B.Cu") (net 3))
 (segment (start 216.4225 77.895) (end 220.5125 81.985) (width 0.2) (layer "B.Cu") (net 3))
 (segment (start 183.365 81.985) (end 187.455 77.895) (width 0.2) (layer "B.Cu") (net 3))
 (segment (start 187.455 77.895) (end 216.4225 77.895) (width 0.2) (layer "B.Cu") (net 3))
 (segment (start 220.5125 101.075) (end 220.5125 92.145) (width 0.2) (layer "F.Cu") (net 10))
 (segment (start 232.5125 103.575) (end 235.0125 101.075) (width 0.2) (layer "F.Cu") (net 12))
 (segment (start 234.0125 100.075) (end 234.0125 81.185) (width 0.2) (layer "F.Cu") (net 12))
 (segment (start 234.0125 81.185) (end 235.7525 79.445) (width 0.2) (layer "F.Cu") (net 12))
 (segment (start 220.5125 103.575) (end 232.5125 103.575) (width 0.2) (layer "F.Cu") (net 12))
 (segment (start 235.0125 101.075) (end 234.0125 100.075) (width 0.2) (layer "F.Cu") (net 12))
 (segment (start 237.9075 91.28) (end 236.2325 89.605) (width 0.2) (layer "F.Cu") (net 13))
 (segment (start 235.0125 106.075) (end 237.9075 103.18) (width 0.2) (layer "F.Cu") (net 13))
 (segment (start 237.9075 103.18) (end 237.9075 91.28) (width 0.2) (layer "F.Cu") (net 13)))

